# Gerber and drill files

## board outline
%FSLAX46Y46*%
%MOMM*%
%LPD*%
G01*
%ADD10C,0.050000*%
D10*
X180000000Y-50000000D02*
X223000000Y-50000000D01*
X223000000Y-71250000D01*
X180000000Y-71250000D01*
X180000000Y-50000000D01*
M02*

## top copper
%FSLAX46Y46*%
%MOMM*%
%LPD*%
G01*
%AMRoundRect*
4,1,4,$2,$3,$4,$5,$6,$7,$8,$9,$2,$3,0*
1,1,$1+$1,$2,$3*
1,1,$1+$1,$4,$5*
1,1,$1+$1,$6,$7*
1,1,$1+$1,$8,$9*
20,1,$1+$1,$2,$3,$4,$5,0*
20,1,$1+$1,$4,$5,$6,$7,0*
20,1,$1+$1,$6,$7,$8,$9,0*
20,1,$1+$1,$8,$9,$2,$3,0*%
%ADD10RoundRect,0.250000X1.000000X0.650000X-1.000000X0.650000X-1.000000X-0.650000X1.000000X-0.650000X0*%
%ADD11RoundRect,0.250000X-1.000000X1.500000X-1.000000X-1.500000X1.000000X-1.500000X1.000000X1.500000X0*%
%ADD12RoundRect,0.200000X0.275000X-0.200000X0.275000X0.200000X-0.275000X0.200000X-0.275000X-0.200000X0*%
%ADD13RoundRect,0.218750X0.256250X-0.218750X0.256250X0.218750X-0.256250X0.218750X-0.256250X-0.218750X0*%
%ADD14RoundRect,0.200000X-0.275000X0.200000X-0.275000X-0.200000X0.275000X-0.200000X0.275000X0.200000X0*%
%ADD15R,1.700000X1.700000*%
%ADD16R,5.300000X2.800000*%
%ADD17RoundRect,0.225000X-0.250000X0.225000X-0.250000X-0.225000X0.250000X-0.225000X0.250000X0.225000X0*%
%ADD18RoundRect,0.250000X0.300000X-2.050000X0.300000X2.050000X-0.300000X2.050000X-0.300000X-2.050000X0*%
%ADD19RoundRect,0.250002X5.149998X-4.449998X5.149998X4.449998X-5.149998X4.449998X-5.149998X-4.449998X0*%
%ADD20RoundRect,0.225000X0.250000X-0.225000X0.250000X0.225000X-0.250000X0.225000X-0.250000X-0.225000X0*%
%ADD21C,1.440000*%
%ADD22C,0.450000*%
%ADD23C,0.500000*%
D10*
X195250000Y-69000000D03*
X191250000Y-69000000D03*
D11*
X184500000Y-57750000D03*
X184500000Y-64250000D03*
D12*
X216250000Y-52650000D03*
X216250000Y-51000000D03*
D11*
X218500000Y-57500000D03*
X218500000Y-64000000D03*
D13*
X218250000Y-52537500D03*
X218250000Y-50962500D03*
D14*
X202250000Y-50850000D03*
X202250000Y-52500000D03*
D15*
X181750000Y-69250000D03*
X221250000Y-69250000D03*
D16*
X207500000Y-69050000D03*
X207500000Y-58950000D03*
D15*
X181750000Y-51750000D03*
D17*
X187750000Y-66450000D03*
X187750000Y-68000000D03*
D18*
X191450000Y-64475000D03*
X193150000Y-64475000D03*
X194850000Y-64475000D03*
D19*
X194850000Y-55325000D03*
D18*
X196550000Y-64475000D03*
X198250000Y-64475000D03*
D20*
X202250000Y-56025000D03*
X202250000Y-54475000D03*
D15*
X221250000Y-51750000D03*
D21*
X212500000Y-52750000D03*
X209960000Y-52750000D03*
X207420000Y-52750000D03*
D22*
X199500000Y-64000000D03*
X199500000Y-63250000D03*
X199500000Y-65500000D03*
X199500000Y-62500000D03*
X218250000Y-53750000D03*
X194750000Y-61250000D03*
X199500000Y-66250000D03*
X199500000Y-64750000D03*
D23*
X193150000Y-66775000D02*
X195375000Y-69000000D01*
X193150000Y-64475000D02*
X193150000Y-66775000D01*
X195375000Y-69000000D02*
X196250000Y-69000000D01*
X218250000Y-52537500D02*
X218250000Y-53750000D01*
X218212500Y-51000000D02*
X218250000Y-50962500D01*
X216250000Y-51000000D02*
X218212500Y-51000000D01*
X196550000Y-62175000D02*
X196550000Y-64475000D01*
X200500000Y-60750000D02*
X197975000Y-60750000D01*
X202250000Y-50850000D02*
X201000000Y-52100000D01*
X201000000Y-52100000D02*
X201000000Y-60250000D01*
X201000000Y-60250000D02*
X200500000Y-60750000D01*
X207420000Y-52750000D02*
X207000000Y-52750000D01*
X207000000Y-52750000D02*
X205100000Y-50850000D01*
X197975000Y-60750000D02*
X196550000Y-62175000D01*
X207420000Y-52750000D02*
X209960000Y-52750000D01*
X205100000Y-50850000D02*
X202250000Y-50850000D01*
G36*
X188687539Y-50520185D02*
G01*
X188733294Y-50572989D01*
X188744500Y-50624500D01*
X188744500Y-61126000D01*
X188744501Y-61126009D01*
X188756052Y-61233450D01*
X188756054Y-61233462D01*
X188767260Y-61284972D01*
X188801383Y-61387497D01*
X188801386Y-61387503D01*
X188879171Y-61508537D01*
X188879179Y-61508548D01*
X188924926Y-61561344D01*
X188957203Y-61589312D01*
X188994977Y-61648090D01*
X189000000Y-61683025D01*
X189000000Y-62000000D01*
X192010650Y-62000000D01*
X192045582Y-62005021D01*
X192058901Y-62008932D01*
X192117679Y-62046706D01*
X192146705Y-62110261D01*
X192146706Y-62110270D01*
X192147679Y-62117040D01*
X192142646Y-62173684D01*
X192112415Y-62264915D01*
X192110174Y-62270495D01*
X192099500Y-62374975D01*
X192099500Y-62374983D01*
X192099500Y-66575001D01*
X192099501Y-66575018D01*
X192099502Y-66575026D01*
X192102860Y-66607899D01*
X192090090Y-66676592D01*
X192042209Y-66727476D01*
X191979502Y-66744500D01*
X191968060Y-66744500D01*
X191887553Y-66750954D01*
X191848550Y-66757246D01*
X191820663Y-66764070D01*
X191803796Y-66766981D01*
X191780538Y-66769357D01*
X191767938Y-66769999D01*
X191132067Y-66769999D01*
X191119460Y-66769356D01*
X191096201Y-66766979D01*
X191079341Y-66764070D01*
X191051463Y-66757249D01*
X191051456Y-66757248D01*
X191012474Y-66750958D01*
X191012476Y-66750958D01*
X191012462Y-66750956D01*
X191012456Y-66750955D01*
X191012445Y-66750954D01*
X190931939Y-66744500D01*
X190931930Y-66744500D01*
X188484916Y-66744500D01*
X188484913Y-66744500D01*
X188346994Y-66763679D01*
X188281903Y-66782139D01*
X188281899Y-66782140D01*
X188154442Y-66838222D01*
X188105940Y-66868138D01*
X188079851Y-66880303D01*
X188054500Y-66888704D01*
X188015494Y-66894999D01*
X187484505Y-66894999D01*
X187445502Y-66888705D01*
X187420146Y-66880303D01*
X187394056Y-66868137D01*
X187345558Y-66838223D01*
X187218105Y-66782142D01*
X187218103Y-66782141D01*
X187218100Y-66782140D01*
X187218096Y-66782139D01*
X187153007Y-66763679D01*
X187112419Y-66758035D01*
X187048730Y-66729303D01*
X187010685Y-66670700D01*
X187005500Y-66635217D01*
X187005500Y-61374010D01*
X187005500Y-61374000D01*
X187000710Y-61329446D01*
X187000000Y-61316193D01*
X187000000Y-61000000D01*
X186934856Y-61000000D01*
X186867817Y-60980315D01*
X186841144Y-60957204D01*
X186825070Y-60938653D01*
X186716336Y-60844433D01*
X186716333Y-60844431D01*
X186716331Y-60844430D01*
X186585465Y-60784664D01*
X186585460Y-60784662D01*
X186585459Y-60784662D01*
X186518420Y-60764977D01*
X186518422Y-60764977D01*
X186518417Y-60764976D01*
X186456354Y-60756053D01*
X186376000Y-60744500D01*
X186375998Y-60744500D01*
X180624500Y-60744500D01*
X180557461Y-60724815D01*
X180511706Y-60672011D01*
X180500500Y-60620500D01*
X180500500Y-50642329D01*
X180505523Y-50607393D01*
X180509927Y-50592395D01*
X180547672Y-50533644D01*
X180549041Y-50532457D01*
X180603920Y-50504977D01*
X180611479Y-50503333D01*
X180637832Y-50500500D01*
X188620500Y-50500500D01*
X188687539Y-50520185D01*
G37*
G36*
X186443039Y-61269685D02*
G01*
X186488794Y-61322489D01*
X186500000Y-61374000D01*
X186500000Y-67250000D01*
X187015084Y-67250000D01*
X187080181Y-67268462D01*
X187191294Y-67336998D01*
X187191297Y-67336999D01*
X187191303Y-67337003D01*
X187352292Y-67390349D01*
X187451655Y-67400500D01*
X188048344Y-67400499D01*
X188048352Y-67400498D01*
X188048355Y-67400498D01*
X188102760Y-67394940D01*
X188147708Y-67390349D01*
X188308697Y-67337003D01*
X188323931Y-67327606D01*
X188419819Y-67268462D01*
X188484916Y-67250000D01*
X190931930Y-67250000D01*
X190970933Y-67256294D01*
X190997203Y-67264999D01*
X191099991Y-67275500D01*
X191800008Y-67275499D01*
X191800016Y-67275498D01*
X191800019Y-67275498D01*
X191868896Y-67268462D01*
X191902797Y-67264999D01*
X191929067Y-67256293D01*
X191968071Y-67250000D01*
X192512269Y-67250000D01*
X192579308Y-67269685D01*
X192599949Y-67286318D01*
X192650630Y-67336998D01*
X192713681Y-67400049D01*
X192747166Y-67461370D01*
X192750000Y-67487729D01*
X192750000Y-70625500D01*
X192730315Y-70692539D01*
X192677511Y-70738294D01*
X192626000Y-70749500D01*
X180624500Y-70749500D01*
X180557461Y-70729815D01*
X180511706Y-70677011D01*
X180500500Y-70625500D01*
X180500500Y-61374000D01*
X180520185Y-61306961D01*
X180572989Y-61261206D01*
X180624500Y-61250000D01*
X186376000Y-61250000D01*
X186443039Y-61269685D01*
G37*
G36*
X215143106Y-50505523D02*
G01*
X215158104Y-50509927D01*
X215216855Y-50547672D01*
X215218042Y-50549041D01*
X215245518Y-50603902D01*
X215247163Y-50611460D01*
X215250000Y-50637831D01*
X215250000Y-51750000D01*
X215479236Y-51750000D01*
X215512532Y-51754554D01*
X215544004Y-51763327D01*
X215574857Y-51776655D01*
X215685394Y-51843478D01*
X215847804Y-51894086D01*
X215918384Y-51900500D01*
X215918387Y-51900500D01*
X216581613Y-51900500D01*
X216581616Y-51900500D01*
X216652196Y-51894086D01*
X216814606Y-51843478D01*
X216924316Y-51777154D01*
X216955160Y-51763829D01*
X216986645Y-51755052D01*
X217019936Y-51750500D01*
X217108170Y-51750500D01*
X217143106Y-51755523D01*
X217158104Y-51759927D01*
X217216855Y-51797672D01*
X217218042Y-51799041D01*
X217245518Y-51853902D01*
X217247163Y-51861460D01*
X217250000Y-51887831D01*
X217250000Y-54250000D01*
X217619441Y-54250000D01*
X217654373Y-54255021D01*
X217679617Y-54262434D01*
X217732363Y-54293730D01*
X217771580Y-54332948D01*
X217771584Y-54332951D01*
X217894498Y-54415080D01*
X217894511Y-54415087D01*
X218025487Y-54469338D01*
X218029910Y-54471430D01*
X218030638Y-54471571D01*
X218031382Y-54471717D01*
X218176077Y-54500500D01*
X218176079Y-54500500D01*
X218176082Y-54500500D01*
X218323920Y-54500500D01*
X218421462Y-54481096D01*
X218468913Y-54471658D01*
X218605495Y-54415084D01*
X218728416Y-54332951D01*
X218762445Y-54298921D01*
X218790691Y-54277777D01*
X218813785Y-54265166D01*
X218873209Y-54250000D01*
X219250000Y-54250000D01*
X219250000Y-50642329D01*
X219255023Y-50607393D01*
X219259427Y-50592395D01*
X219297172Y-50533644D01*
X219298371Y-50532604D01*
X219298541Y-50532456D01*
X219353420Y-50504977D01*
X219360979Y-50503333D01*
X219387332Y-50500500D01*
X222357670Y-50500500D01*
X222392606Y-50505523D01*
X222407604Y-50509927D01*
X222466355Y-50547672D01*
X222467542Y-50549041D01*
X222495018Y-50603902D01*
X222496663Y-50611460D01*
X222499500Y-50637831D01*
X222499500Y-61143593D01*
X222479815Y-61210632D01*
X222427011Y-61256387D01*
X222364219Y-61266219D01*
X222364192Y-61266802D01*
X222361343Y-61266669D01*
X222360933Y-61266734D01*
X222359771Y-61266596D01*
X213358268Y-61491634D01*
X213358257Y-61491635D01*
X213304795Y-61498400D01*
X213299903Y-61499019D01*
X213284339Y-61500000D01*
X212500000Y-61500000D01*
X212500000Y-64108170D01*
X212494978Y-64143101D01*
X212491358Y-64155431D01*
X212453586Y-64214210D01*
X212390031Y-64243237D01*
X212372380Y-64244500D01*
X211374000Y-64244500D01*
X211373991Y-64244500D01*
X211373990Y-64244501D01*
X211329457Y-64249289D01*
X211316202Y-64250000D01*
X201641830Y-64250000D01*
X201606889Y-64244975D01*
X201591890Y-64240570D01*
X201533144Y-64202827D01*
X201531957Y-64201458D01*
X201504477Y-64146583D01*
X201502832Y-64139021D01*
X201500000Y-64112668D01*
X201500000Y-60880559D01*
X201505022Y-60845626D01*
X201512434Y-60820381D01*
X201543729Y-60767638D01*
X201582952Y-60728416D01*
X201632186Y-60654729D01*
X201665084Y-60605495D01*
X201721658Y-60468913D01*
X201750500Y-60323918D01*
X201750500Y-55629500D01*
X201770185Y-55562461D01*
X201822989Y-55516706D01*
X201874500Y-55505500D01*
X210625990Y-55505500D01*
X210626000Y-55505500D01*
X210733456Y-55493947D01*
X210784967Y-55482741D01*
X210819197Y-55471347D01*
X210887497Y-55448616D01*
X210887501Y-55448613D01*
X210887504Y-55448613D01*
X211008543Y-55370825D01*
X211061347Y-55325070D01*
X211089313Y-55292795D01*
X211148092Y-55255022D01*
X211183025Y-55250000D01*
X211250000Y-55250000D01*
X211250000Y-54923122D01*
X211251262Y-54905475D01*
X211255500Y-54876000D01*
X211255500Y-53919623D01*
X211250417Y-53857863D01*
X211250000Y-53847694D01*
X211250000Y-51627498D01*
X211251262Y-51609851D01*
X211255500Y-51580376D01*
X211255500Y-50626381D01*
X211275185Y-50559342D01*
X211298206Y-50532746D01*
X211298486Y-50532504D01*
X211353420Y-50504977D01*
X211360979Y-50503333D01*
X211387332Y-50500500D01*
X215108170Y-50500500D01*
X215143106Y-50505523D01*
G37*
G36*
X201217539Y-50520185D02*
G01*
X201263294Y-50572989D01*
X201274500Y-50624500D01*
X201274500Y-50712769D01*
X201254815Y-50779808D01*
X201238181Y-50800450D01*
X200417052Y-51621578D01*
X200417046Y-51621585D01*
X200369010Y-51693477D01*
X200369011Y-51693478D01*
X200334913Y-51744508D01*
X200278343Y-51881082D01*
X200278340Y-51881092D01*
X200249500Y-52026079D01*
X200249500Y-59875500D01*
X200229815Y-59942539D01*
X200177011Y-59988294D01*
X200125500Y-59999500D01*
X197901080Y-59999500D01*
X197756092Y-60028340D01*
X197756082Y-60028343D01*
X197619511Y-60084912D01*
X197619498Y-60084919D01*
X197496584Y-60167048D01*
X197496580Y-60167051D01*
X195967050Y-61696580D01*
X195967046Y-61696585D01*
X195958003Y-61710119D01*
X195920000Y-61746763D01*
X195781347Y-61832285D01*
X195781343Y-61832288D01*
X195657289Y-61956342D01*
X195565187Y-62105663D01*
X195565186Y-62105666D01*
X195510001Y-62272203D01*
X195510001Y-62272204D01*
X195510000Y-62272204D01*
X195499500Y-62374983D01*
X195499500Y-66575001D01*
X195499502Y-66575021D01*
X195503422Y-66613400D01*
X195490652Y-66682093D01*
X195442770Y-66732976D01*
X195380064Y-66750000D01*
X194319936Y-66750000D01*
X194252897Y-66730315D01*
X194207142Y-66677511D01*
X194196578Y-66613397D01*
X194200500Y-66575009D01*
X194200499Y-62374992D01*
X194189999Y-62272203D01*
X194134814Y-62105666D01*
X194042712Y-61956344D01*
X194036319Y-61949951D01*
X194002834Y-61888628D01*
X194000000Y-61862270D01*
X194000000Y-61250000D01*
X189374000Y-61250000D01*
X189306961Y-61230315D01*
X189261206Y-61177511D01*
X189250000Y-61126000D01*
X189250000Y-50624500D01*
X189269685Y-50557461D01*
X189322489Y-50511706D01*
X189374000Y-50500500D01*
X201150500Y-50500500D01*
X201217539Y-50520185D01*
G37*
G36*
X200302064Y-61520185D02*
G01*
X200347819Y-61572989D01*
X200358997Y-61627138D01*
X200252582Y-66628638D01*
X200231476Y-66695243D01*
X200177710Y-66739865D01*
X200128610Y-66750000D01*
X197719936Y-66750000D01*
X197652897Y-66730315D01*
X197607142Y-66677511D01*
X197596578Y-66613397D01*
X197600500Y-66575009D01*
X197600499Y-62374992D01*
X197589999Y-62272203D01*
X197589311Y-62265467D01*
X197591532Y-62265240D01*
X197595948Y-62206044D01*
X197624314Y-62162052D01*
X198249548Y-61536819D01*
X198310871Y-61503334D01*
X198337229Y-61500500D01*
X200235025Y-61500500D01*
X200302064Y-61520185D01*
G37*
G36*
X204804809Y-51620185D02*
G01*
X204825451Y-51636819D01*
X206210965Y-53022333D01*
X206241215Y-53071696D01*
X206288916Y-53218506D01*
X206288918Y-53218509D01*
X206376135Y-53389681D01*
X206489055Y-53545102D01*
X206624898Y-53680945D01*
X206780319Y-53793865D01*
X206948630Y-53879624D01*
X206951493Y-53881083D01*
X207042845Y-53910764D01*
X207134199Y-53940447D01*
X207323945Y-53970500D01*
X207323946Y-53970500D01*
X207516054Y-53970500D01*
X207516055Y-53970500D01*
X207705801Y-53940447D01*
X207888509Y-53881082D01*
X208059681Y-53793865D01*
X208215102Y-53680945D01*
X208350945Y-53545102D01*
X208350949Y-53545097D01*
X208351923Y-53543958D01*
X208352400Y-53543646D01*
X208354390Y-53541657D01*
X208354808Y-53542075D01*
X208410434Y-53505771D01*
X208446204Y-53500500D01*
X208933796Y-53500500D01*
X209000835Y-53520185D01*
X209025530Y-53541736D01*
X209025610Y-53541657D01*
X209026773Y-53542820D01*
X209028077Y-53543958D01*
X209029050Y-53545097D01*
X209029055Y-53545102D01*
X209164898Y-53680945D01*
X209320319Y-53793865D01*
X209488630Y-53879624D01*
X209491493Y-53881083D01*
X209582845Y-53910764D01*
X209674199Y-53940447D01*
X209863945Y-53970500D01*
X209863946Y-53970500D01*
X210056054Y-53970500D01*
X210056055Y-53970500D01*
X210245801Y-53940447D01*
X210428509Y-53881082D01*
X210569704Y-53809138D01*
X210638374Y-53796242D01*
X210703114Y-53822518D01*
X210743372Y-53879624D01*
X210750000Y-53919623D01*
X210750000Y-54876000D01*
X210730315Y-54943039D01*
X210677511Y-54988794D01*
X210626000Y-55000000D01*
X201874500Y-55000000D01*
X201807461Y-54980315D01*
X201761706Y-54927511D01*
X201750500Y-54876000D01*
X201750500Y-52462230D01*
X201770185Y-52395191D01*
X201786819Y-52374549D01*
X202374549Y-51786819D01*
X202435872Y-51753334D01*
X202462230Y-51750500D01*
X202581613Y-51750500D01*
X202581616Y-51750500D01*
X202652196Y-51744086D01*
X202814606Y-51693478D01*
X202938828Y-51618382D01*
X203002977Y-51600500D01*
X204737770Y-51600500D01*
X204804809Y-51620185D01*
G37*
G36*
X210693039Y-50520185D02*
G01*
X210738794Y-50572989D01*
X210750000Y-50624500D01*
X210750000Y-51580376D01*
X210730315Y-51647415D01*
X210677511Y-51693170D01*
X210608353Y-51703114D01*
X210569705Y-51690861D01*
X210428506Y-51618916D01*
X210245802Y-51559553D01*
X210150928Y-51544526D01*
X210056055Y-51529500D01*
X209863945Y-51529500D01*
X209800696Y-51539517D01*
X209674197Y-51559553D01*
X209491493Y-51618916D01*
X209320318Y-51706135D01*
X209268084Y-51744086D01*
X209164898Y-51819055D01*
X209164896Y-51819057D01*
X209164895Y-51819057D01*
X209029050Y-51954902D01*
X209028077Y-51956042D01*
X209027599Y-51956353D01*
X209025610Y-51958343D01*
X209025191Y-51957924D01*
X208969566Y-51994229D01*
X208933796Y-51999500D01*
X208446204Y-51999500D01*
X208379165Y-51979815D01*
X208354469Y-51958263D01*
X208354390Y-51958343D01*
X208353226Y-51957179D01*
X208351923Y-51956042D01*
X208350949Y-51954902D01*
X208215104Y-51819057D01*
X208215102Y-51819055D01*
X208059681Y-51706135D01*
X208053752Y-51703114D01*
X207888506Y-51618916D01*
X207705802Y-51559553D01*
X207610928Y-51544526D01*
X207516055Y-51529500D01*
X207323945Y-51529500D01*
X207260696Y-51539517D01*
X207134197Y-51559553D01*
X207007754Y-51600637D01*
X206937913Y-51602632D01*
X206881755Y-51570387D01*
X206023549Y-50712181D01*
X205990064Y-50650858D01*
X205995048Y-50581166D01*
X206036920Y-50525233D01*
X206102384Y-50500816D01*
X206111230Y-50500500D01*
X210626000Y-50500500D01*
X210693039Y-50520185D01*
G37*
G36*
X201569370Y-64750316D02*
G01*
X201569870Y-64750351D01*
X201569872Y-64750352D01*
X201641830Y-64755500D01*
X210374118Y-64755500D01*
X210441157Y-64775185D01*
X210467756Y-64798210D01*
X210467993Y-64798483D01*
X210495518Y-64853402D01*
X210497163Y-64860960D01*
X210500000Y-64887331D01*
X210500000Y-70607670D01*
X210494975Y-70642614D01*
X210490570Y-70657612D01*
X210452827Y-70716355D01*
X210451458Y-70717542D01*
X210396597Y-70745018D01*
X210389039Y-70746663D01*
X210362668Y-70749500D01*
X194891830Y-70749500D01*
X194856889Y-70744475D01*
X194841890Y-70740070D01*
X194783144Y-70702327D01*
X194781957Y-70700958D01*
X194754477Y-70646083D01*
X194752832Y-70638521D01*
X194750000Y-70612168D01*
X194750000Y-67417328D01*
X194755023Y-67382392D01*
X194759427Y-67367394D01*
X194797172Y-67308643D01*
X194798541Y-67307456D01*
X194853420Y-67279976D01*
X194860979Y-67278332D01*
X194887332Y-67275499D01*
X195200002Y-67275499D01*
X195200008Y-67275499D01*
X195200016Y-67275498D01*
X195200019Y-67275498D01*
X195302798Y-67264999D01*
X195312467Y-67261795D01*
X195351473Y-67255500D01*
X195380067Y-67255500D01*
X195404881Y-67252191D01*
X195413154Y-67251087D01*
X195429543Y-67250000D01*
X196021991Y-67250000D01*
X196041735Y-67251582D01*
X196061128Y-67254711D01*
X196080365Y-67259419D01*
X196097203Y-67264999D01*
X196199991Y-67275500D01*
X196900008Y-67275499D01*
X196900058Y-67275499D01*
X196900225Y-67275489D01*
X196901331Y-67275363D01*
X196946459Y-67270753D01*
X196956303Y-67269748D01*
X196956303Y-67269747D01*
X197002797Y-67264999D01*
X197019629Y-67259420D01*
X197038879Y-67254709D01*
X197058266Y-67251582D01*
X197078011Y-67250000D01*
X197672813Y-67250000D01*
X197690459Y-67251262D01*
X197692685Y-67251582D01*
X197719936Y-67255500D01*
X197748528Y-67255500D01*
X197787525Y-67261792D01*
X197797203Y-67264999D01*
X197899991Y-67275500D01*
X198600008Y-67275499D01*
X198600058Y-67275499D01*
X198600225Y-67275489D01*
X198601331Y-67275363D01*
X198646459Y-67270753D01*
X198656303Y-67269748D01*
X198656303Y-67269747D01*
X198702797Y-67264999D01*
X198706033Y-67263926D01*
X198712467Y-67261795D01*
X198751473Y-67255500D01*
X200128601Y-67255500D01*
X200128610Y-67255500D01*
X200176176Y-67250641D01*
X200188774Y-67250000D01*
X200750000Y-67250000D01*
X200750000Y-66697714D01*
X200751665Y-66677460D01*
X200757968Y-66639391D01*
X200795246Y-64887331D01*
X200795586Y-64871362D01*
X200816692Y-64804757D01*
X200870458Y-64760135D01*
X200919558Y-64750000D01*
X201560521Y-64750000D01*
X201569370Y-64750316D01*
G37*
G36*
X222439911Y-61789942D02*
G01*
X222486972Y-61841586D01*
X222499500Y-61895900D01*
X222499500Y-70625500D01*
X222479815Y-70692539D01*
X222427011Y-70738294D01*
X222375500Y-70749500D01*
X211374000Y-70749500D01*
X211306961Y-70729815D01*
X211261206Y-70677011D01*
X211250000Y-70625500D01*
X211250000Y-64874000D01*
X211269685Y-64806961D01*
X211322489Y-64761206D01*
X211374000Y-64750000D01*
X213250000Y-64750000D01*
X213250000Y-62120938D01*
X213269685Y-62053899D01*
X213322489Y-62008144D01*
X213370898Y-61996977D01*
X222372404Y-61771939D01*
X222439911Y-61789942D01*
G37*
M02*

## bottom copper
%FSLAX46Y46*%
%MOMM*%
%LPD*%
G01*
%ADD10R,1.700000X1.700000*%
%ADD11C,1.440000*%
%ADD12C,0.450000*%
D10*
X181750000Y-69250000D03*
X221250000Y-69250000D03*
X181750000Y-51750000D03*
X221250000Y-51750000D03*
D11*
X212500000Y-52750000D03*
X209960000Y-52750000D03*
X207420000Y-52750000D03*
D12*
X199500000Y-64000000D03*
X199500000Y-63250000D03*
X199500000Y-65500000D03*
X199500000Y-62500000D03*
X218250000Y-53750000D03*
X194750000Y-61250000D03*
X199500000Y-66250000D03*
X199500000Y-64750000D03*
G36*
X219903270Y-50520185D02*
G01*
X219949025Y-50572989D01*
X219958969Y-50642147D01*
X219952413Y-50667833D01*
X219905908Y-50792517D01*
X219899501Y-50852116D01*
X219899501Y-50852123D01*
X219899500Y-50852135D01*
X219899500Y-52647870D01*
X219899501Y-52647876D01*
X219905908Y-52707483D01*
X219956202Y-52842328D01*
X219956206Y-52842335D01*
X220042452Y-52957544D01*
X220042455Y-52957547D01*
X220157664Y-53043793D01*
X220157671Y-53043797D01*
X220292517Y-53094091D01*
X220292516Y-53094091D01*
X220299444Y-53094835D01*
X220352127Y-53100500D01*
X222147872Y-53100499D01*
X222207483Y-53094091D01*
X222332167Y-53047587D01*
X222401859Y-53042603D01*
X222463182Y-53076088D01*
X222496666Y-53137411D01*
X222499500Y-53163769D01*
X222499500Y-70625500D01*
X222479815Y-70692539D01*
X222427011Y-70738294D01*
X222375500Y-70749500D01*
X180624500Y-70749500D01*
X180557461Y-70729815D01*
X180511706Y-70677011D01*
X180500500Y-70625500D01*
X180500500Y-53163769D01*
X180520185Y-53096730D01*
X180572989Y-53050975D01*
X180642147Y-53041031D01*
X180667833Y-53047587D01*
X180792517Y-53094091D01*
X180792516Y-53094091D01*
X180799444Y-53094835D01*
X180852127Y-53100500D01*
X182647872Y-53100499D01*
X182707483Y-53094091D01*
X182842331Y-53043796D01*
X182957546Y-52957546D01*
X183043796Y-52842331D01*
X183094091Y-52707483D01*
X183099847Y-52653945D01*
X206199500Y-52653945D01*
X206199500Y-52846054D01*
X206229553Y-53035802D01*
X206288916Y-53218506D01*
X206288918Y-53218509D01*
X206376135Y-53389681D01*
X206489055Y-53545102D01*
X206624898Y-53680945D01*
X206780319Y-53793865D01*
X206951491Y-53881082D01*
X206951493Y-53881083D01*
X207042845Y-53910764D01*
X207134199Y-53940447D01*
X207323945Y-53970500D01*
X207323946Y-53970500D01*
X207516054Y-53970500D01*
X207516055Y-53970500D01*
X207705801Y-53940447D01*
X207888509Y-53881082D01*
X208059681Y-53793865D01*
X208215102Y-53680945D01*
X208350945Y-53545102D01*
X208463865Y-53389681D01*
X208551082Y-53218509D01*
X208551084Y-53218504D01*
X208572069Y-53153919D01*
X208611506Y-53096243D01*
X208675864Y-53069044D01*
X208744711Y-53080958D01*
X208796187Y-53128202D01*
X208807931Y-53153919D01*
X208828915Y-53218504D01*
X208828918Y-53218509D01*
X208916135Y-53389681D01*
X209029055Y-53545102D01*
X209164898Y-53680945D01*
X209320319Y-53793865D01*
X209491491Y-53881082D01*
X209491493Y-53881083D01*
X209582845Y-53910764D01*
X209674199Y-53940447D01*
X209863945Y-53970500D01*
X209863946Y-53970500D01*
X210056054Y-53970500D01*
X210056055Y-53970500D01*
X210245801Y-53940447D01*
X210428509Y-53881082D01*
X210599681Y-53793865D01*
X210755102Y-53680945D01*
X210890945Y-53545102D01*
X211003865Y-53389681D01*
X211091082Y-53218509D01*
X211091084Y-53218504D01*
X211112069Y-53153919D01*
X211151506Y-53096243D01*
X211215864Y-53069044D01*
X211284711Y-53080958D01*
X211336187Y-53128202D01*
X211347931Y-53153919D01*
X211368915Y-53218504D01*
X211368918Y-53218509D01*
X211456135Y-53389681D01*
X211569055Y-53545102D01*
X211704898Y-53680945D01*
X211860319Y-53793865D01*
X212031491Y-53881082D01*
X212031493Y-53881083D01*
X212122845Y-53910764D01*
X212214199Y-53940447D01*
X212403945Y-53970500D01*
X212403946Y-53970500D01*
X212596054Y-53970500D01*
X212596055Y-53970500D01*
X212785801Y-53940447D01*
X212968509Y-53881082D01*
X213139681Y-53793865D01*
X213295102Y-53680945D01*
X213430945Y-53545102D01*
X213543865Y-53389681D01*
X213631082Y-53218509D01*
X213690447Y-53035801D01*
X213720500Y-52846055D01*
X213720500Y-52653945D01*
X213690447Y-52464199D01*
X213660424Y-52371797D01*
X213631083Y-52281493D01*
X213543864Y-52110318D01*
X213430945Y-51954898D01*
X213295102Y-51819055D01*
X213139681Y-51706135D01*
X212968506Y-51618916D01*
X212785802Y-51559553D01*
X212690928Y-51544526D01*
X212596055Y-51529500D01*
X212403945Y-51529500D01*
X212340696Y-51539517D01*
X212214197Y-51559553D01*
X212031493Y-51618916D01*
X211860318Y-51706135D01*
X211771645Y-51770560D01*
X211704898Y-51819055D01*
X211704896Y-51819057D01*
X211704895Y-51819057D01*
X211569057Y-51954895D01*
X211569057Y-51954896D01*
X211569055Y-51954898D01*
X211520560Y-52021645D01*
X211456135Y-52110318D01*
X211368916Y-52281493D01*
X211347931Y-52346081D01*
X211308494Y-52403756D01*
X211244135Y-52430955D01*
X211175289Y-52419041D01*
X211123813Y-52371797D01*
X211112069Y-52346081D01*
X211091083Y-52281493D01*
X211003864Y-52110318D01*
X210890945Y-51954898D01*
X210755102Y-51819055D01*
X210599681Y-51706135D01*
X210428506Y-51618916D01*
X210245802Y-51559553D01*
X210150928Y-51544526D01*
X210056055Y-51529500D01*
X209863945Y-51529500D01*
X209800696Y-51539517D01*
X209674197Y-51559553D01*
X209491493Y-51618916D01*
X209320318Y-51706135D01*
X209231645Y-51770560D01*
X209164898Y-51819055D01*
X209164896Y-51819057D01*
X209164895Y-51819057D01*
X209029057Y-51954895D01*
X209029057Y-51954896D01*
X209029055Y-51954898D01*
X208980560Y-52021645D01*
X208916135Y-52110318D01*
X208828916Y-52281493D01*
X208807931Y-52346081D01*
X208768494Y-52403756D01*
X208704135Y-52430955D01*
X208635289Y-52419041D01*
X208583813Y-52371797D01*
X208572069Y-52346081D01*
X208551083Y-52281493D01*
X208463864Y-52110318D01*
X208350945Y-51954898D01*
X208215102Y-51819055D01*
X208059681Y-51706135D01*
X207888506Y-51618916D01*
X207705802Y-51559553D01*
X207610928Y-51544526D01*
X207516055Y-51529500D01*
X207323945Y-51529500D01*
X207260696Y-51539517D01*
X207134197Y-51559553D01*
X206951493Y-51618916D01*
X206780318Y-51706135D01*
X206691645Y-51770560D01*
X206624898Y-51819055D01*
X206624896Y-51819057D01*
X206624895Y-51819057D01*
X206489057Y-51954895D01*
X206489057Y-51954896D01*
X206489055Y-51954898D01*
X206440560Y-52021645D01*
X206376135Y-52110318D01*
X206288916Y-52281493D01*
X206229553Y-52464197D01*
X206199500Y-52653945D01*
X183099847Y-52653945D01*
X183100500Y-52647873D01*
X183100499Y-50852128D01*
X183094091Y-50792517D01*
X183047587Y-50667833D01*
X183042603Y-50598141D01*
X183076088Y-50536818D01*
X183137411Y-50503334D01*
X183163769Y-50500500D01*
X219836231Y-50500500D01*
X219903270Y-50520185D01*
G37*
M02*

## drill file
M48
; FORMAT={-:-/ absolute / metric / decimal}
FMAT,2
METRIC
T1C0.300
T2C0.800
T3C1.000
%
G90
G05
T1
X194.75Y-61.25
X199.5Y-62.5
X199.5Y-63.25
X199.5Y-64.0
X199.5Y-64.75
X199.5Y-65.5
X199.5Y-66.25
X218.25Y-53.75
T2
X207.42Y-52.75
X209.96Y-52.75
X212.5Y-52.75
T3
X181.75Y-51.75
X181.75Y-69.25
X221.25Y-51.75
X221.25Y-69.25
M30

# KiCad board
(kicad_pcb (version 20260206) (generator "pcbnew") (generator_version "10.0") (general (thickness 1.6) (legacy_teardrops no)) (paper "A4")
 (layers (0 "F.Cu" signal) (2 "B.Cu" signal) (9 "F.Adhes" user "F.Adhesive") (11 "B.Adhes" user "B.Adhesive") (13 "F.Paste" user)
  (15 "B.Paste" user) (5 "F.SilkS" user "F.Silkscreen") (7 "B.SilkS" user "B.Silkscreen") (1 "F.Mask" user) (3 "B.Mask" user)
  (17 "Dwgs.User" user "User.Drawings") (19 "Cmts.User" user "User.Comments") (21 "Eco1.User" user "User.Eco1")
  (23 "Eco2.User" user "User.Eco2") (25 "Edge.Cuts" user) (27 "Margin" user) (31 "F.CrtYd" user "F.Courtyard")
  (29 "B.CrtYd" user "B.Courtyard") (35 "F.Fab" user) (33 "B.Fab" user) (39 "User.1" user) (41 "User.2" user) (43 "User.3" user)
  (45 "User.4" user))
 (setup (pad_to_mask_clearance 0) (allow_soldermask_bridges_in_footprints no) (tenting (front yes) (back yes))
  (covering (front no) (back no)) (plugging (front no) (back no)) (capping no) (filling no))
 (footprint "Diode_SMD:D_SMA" (layer "F.Cu") (at 193.25 69 180)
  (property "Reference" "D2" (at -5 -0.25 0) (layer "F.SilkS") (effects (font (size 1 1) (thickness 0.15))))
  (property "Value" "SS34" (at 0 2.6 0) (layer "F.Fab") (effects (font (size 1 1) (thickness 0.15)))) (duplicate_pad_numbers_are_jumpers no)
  (pad "1" smd roundrect (at -2 0 180) (size 2.5 1.8) (layers "F.Cu" "F.Mask" "F.Paste") (roundrect_rratio 0.1388888889) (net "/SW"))
  (pad "2" smd roundrect (at 2 0 180) (size 2.5 1.8) (layers "F.Cu" "F.Mask" "F.Paste") (roundrect_rratio 0.1388888889) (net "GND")))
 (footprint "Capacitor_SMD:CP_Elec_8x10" (layer "F.Cu") (at 184.5 61 -90)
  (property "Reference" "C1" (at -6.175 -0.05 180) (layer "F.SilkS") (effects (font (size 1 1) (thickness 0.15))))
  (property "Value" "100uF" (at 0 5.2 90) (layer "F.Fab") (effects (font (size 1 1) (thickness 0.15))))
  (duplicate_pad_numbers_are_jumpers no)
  (pad "1" smd roundrect (at -3.25 0 270) (size 3.5 2.5) (layers "F.Cu" "F.Mask" "F.Paste") (roundrect_rratio 0.1) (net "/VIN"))
  (pad "2" smd roundrect (at 3.25 0 270) (size 3.5 2.5) (layers "F.Cu" "F.Mask" "F.Paste") (roundrect_rratio 0.1) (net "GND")))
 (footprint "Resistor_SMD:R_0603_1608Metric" (layer "F.Cu") (at 216.25 51.825 90)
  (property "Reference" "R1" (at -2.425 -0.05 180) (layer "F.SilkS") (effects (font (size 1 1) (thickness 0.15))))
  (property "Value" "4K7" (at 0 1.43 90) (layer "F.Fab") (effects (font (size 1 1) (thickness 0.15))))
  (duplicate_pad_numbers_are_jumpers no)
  (pad "1" smd roundrect (at -0.825 0 90) (size 0.8 0.95) (layers "F.Cu" "F.Mask" "F.Paste") (roundrect_rratio 0.25) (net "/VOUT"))
  (pad "2" smd roundrect (at 0.825 0 90) (size 0.8 0.95) (layers "F.Cu" "F.Mask" "F.Paste") (roundrect_rratio 0.25) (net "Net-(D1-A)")))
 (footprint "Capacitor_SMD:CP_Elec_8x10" (layer "F.Cu") (at 218.5 60.75 -90)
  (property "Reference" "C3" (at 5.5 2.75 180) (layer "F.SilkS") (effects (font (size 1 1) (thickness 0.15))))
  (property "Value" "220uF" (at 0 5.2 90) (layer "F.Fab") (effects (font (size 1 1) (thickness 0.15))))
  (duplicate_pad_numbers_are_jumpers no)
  (pad "1" smd roundrect (at -3.25 0 270) (size 3.5 2.5) (layers "F.Cu" "F.Mask" "F.Paste") (roundrect_rratio 0.1) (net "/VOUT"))
  (pad "2" smd roundrect (at 3.25 0 270) (size 3.5 2.5) (layers "F.Cu" "F.Mask" "F.Paste") (roundrect_rratio 0.1) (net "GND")))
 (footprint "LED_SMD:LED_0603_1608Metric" (layer "F.Cu") (at 218.25 51.75 90)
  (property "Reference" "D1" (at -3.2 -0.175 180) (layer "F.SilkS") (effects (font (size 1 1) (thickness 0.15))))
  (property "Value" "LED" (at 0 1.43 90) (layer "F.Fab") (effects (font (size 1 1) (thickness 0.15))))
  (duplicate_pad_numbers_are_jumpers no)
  (pad "1" smd roundrect (at -0.7875 0 90) (size 0.875 0.95) (layers "F.Cu" "F.Mask" "F.Paste") (roundrect_rratio 0.25) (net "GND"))
  (pad "2" smd roundrect (at 0.7875 0 90) (size 0.875 0.95) (layers "F.Cu" "F.Mask" "F.Paste") (roundrect_rratio 0.25) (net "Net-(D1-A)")))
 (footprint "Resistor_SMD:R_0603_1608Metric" (layer "F.Cu") (at 202.25 51.675 -90)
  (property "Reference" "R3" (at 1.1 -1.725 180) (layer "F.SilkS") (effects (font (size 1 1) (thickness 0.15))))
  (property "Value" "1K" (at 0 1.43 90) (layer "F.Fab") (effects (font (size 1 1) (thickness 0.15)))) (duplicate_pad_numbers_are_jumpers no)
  (pad "1" smd roundrect (at -0.825 0 270) (size 0.8 0.95) (layers "F.Cu" "F.Mask" "F.Paste") (roundrect_rratio 0.25) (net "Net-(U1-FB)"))
  (pad "2" smd roundrect (at 0.825 0 270) (size 0.8 0.95) (layers "F.Cu" "F.Mask" "F.Paste") (roundrect_rratio 0.25) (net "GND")))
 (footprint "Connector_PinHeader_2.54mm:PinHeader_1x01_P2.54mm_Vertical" (layer "F.Cu") (at 181.75 69.25)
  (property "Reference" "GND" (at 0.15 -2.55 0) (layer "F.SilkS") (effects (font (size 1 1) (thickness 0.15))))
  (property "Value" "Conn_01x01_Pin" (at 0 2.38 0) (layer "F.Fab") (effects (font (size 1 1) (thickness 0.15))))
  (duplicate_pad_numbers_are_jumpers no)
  (pad "1" thru_hole rect (at 0 0) (size 1.7 1.7) (drill 1) (layers "*.Cu" "*.Mask") (remove_unused_layers no) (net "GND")))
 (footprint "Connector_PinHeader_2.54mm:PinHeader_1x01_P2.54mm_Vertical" (layer "F.Cu") (at 221.25 69.25)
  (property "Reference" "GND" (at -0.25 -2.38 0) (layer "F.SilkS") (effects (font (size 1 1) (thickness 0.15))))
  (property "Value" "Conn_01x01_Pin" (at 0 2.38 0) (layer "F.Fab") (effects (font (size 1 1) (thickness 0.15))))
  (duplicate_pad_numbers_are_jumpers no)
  (pad "1" thru_hole rect (at 0 0) (size 1.7 1.7) (drill 1) (layers "*.Cu" "*.Mask") (remove_unused_layers no) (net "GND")))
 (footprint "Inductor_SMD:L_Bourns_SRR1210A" (layer "F.Cu") (at 207.5 64 90)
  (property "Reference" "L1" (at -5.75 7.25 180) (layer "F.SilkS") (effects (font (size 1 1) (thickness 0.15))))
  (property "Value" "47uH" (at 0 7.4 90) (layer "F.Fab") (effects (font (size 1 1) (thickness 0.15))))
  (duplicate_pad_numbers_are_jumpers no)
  (pad "1" smd rect (at -5.05 0 90) (size 2.8 5.3) (layers "F.Cu" "F.Mask" "F.Paste") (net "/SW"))
  (pad "2" smd rect (at 5.05 0 90) (size 2.8 5.3) (layers "F.Cu" "F.Mask" "F.Paste") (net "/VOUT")))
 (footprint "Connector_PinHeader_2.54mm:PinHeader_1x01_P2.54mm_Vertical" (layer "F.Cu") (at 181.75 51.75)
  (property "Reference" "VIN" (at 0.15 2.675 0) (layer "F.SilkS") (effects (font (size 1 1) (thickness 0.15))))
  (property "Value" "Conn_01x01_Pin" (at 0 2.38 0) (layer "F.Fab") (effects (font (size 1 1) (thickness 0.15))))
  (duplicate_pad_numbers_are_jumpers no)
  (pad "1" thru_hole rect (at 0 0) (size 1.7 1.7) (drill 1) (layers "*.Cu" "*.Mask") (remove_unused_layers no) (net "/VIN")))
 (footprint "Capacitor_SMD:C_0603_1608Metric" (layer "F.Cu") (at 187.75 67.225 -90)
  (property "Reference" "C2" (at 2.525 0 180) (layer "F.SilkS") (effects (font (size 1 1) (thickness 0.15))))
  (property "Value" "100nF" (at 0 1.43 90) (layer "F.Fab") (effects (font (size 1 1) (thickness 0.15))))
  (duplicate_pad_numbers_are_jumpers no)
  (pad "1" smd roundrect (at -0.775 0 270) (size 0.9 0.95) (layers "F.Cu" "F.Mask" "F.Paste") (roundrect_rratio 0.25) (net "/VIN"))
  (pad "2" smd roundrect (at 0.775 0 270) (size 0.9 0.95) (layers "F.Cu" "F.Mask" "F.Paste") (roundrect_rratio 0.25) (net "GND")))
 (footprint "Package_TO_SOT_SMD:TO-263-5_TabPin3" (layer "F.Cu") (at 194.85 56.825 90)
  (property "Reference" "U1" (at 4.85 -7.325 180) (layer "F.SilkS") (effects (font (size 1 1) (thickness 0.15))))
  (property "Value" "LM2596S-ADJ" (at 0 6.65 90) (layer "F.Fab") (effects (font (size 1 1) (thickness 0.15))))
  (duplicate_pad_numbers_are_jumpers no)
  (pad "" smd roundrect (at -0.925 -2.775 90) (size 4.55 5.25) (layers "F.Paste") (roundrect_rratio 0.054945))
  (pad "" smd roundrect (at -0.925 2.775 90) (size 4.55 5.25) (layers "F.Paste") (roundrect_rratio 0.054945))
  (pad "" smd roundrect (at 3.925 -2.775 90) (size 4.55 5.25) (layers "F.Paste") (roundrect_rratio 0.054945))
  (pad "" smd roundrect (at 3.925 2.775 90) (size 4.55 5.25) (layers "F.Paste") (roundrect_rratio 0.054945))
  (pad "1" smd roundrect (at -7.65 -3.4 90) (size 4.6 1.1) (layers "F.Cu" "F.Mask" "F.Paste") (roundrect_rratio 0.227273) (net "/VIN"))
  (pad "2" smd roundrect (at -7.65 -1.7 90) (size 4.6 1.1) (layers "F.Cu" "F.Mask" "F.Paste") (roundrect_rratio 0.227273) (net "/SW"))
  (pad "3" smd roundrect (at -7.65 0 90) (size 4.6 1.1) (layers "F.Cu" "F.Mask" "F.Paste") (roundrect_rratio 0.227273) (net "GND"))
  (pad "3" smd roundrect (at 1.5 0 90) (size 9.4 10.8) (layers "F.Cu" "F.Mask") (roundrect_rratio 0.026596) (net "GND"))
  (pad "4" smd roundrect (at -7.65 1.7 90) (size 4.6 1.1) (layers "F.Cu" "F.Mask" "F.Paste") (roundrect_rratio 0.227273) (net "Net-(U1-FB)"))
  (pad "5" smd roundrect (at -7.65 3.4 90) (size 4.6 1.1) (layers "F.Cu" "F.Mask" "F.Paste") (roundrect_rratio 0.227273) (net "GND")))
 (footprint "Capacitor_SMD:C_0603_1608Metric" (layer "F.Cu") (at 202.25 55.25 90)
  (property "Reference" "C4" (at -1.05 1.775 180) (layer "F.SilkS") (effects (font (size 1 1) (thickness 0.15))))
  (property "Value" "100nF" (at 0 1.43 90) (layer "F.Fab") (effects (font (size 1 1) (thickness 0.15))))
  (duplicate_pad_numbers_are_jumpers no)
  (pad "1" smd roundrect (at -0.775 0 90) (size 0.9 0.95) (layers "F.Cu" "F.Mask" "F.Paste") (roundrect_rratio 0.25) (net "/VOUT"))
  (pad "2" smd roundrect (at 0.775 0 90) (size 0.9 0.95) (layers "F.Cu" "F.Mask" "F.Paste") (roundrect_rratio 0.25) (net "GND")))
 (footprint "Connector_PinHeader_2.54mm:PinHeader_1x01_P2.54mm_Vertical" (layer "F.Cu") (at 221.25 51.75)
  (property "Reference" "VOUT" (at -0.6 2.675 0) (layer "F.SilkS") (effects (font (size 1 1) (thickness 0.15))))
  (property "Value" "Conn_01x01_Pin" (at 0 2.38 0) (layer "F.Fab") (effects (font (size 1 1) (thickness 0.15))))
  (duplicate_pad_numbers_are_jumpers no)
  (pad "1" thru_hole rect (at 0 0) (size 1.7 1.7) (drill 1) (layers "*.Cu" "*.Mask") (remove_unused_layers no) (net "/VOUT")))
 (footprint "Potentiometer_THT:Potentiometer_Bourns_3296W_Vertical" (layer "F.Cu") (at 212.5 52.75)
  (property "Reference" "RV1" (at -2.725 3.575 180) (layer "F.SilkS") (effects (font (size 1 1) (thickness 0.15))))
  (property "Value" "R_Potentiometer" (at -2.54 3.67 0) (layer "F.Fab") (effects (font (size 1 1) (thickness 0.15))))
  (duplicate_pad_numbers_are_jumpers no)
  (pad "1" thru_hole circle (at 0 0) (size 1.44 1.44) (drill 0.8) (layers "*.Cu" "*.Mask") (remove_unused_layers no) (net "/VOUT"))
  (pad "2" thru_hole circle (at -2.54 0) (size 1.44 1.44) (drill 0.8) (layers "*.Cu" "*.Mask") (remove_unused_layers no) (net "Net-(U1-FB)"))
  (pad "3" thru_hole circle (at -5.08 0) (size 1.44 1.44) (drill 0.8) (layers "*.Cu" "*.Mask") (remove_unused_layers no) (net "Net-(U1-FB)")))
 (gr_rect (start 180 50) (end 223 71.25) (stroke (width 0.05) (type default)) (fill no) (layer "Edge.Cuts"))
 (segment (start 193.15 66.775) (end 195.375 69) (width 0.5) (layer "F.Cu") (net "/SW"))
 (segment (start 193.15 64.475) (end 193.15 66.775) (width 0.5) (layer "F.Cu") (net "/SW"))
 (segment (start 195.375 69) (end 196.25 69) (width 0.5) (layer "F.Cu") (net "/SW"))
 (segment (start 218.25 52.5375) (end 218.25 53.75) (width 0.5) (layer "F.Cu") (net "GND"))
 (via (at 199.5 64) (size 0.45) (drill 0.3) (layers "F.Cu" "B.Cu") (free yes) (capping no) (covering (front no) (back no))
  (plugging (front no) (back no)) (filling no) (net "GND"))
 (via (at 199.5 63.25) (size 0.45) (drill 0.3) (layers "F.Cu" "B.Cu") (free yes) (capping no) (covering (front no) (back no))
  (plugging (front no) (back no)) (filling no) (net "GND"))
 (via (at 199.5 65.5) (size 0.45) (drill 0.3) (layers "F.Cu" "B.Cu") (free yes) (capping no) (covering (front no) (back no))
  (plugging (front no) (back no)) (filling no) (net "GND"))
 (via (at 199.5 62.5) (size 0.45) (drill 0.3) (layers "F.Cu" "B.Cu") (free yes) (capping no) (covering (front no) (back no))
  (plugging (front no) (back no)) (filling no) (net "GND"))
 (via (at 218.25 53.75) (size 0.45) (drill 0.3) (layers "F.Cu" "B.Cu") (capping no) (covering (front no) (back no))
  (plugging (front no) (back no)) (filling no) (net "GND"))
 (via (at 194.75 61.25) (size 0.45) (drill 0.3) (layers "F.Cu" "B.Cu") (free yes) (capping no) (covering (front no) (back no))
  (plugging (front no) (back no)) (filling no) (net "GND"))
 (via (at 199.5 66.25) (size 0.45) (drill 0.3) (layers "F.Cu" "B.Cu") (free yes) (capping no) (covering (front no) (back no))
  (plugging (front no) (back no)) (filling no) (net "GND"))
 (via (at 199.5 64.75) (size 0.45) (drill 0.3) (layers "F.Cu" "B.Cu") (free yes) (capping no) (covering (front no) (back no))
  (plugging (front no) (back no)) (filling no) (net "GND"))
 (segment (start 218.2125 51) (end 218.25 50.9625) (width 0.5) (layer "F.Cu") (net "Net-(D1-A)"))
 (segment (start 216.25 51) (end 218.2125 51) (width 0.5) (layer "F.Cu") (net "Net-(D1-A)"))
 (segment (start 196.55 62.175) (end 196.55 64.475) (width 0.5) (layer "F.Cu") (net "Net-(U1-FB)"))
 (segment (start 200.5 60.75) (end 197.975 60.75) (width 0.5) (layer "F.Cu") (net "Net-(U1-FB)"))
 (segment (start 202.25 50.85) (end 201 52.1) (width 0.5) (layer "F.Cu") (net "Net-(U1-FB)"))
 (segment (start 201 52.1) (end 201 60.25) (width 0.5) (layer "F.Cu") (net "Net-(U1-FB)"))
 (segment (start 201 60.25) (end 200.5 60.75) (width 0.5) (layer "F.Cu") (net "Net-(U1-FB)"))
 (segment (start 207.42 52.75) (end 207 52.75) (width 0.5) (layer "F.Cu") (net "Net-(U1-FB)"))
 (segment (start 207 52.75) (end 205.1 50.85) (width 0.5) (layer "F.Cu") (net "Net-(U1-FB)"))
 (segment (start 197.975 60.75) (end 196.55 62.175) (width 0.5) (layer "F.Cu") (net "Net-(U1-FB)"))
 (segment (start 207.42 52.75) (end 209.96 52.75) (width 0.5) (layer "F.Cu") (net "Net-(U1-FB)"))
 (segment (start 205.1 50.85) (end 202.25 50.85) (width 0.5) (layer "F.Cu") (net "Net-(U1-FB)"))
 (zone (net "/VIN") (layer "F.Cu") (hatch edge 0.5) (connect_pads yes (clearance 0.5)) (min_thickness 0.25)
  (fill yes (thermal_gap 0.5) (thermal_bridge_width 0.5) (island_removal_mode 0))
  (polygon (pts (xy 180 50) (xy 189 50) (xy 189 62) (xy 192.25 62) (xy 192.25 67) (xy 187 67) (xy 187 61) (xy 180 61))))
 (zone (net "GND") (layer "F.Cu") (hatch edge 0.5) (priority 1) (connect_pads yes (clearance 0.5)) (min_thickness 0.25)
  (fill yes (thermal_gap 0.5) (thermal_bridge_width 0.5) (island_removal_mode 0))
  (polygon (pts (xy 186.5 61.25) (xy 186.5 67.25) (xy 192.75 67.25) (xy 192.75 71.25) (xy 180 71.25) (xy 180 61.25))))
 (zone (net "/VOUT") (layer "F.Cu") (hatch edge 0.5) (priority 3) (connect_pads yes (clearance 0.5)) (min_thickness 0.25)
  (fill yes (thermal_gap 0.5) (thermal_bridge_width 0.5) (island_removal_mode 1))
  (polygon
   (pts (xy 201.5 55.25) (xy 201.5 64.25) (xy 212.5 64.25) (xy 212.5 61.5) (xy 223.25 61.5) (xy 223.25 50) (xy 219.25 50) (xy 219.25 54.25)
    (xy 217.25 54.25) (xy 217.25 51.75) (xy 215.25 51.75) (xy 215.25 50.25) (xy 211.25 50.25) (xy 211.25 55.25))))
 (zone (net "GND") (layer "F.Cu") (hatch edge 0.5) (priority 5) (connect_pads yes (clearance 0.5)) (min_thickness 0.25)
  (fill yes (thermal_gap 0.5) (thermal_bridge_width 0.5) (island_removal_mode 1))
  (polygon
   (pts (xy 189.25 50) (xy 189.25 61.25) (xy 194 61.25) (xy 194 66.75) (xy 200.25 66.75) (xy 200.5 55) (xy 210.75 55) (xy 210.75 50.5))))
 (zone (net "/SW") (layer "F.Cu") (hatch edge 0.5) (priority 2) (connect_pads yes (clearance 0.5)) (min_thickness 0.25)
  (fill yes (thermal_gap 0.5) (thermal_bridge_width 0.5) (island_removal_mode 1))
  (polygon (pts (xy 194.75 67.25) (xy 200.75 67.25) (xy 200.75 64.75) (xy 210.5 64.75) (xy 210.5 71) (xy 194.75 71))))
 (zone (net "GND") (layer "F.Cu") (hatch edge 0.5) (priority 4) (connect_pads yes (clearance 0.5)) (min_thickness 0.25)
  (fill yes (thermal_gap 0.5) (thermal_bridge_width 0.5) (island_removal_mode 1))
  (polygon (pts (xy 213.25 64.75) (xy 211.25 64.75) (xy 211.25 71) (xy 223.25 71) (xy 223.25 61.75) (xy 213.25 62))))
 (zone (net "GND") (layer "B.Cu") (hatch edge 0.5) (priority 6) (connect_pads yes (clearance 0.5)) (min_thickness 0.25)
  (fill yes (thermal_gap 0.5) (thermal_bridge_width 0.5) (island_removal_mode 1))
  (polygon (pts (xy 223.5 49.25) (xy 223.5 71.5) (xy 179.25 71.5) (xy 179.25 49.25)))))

